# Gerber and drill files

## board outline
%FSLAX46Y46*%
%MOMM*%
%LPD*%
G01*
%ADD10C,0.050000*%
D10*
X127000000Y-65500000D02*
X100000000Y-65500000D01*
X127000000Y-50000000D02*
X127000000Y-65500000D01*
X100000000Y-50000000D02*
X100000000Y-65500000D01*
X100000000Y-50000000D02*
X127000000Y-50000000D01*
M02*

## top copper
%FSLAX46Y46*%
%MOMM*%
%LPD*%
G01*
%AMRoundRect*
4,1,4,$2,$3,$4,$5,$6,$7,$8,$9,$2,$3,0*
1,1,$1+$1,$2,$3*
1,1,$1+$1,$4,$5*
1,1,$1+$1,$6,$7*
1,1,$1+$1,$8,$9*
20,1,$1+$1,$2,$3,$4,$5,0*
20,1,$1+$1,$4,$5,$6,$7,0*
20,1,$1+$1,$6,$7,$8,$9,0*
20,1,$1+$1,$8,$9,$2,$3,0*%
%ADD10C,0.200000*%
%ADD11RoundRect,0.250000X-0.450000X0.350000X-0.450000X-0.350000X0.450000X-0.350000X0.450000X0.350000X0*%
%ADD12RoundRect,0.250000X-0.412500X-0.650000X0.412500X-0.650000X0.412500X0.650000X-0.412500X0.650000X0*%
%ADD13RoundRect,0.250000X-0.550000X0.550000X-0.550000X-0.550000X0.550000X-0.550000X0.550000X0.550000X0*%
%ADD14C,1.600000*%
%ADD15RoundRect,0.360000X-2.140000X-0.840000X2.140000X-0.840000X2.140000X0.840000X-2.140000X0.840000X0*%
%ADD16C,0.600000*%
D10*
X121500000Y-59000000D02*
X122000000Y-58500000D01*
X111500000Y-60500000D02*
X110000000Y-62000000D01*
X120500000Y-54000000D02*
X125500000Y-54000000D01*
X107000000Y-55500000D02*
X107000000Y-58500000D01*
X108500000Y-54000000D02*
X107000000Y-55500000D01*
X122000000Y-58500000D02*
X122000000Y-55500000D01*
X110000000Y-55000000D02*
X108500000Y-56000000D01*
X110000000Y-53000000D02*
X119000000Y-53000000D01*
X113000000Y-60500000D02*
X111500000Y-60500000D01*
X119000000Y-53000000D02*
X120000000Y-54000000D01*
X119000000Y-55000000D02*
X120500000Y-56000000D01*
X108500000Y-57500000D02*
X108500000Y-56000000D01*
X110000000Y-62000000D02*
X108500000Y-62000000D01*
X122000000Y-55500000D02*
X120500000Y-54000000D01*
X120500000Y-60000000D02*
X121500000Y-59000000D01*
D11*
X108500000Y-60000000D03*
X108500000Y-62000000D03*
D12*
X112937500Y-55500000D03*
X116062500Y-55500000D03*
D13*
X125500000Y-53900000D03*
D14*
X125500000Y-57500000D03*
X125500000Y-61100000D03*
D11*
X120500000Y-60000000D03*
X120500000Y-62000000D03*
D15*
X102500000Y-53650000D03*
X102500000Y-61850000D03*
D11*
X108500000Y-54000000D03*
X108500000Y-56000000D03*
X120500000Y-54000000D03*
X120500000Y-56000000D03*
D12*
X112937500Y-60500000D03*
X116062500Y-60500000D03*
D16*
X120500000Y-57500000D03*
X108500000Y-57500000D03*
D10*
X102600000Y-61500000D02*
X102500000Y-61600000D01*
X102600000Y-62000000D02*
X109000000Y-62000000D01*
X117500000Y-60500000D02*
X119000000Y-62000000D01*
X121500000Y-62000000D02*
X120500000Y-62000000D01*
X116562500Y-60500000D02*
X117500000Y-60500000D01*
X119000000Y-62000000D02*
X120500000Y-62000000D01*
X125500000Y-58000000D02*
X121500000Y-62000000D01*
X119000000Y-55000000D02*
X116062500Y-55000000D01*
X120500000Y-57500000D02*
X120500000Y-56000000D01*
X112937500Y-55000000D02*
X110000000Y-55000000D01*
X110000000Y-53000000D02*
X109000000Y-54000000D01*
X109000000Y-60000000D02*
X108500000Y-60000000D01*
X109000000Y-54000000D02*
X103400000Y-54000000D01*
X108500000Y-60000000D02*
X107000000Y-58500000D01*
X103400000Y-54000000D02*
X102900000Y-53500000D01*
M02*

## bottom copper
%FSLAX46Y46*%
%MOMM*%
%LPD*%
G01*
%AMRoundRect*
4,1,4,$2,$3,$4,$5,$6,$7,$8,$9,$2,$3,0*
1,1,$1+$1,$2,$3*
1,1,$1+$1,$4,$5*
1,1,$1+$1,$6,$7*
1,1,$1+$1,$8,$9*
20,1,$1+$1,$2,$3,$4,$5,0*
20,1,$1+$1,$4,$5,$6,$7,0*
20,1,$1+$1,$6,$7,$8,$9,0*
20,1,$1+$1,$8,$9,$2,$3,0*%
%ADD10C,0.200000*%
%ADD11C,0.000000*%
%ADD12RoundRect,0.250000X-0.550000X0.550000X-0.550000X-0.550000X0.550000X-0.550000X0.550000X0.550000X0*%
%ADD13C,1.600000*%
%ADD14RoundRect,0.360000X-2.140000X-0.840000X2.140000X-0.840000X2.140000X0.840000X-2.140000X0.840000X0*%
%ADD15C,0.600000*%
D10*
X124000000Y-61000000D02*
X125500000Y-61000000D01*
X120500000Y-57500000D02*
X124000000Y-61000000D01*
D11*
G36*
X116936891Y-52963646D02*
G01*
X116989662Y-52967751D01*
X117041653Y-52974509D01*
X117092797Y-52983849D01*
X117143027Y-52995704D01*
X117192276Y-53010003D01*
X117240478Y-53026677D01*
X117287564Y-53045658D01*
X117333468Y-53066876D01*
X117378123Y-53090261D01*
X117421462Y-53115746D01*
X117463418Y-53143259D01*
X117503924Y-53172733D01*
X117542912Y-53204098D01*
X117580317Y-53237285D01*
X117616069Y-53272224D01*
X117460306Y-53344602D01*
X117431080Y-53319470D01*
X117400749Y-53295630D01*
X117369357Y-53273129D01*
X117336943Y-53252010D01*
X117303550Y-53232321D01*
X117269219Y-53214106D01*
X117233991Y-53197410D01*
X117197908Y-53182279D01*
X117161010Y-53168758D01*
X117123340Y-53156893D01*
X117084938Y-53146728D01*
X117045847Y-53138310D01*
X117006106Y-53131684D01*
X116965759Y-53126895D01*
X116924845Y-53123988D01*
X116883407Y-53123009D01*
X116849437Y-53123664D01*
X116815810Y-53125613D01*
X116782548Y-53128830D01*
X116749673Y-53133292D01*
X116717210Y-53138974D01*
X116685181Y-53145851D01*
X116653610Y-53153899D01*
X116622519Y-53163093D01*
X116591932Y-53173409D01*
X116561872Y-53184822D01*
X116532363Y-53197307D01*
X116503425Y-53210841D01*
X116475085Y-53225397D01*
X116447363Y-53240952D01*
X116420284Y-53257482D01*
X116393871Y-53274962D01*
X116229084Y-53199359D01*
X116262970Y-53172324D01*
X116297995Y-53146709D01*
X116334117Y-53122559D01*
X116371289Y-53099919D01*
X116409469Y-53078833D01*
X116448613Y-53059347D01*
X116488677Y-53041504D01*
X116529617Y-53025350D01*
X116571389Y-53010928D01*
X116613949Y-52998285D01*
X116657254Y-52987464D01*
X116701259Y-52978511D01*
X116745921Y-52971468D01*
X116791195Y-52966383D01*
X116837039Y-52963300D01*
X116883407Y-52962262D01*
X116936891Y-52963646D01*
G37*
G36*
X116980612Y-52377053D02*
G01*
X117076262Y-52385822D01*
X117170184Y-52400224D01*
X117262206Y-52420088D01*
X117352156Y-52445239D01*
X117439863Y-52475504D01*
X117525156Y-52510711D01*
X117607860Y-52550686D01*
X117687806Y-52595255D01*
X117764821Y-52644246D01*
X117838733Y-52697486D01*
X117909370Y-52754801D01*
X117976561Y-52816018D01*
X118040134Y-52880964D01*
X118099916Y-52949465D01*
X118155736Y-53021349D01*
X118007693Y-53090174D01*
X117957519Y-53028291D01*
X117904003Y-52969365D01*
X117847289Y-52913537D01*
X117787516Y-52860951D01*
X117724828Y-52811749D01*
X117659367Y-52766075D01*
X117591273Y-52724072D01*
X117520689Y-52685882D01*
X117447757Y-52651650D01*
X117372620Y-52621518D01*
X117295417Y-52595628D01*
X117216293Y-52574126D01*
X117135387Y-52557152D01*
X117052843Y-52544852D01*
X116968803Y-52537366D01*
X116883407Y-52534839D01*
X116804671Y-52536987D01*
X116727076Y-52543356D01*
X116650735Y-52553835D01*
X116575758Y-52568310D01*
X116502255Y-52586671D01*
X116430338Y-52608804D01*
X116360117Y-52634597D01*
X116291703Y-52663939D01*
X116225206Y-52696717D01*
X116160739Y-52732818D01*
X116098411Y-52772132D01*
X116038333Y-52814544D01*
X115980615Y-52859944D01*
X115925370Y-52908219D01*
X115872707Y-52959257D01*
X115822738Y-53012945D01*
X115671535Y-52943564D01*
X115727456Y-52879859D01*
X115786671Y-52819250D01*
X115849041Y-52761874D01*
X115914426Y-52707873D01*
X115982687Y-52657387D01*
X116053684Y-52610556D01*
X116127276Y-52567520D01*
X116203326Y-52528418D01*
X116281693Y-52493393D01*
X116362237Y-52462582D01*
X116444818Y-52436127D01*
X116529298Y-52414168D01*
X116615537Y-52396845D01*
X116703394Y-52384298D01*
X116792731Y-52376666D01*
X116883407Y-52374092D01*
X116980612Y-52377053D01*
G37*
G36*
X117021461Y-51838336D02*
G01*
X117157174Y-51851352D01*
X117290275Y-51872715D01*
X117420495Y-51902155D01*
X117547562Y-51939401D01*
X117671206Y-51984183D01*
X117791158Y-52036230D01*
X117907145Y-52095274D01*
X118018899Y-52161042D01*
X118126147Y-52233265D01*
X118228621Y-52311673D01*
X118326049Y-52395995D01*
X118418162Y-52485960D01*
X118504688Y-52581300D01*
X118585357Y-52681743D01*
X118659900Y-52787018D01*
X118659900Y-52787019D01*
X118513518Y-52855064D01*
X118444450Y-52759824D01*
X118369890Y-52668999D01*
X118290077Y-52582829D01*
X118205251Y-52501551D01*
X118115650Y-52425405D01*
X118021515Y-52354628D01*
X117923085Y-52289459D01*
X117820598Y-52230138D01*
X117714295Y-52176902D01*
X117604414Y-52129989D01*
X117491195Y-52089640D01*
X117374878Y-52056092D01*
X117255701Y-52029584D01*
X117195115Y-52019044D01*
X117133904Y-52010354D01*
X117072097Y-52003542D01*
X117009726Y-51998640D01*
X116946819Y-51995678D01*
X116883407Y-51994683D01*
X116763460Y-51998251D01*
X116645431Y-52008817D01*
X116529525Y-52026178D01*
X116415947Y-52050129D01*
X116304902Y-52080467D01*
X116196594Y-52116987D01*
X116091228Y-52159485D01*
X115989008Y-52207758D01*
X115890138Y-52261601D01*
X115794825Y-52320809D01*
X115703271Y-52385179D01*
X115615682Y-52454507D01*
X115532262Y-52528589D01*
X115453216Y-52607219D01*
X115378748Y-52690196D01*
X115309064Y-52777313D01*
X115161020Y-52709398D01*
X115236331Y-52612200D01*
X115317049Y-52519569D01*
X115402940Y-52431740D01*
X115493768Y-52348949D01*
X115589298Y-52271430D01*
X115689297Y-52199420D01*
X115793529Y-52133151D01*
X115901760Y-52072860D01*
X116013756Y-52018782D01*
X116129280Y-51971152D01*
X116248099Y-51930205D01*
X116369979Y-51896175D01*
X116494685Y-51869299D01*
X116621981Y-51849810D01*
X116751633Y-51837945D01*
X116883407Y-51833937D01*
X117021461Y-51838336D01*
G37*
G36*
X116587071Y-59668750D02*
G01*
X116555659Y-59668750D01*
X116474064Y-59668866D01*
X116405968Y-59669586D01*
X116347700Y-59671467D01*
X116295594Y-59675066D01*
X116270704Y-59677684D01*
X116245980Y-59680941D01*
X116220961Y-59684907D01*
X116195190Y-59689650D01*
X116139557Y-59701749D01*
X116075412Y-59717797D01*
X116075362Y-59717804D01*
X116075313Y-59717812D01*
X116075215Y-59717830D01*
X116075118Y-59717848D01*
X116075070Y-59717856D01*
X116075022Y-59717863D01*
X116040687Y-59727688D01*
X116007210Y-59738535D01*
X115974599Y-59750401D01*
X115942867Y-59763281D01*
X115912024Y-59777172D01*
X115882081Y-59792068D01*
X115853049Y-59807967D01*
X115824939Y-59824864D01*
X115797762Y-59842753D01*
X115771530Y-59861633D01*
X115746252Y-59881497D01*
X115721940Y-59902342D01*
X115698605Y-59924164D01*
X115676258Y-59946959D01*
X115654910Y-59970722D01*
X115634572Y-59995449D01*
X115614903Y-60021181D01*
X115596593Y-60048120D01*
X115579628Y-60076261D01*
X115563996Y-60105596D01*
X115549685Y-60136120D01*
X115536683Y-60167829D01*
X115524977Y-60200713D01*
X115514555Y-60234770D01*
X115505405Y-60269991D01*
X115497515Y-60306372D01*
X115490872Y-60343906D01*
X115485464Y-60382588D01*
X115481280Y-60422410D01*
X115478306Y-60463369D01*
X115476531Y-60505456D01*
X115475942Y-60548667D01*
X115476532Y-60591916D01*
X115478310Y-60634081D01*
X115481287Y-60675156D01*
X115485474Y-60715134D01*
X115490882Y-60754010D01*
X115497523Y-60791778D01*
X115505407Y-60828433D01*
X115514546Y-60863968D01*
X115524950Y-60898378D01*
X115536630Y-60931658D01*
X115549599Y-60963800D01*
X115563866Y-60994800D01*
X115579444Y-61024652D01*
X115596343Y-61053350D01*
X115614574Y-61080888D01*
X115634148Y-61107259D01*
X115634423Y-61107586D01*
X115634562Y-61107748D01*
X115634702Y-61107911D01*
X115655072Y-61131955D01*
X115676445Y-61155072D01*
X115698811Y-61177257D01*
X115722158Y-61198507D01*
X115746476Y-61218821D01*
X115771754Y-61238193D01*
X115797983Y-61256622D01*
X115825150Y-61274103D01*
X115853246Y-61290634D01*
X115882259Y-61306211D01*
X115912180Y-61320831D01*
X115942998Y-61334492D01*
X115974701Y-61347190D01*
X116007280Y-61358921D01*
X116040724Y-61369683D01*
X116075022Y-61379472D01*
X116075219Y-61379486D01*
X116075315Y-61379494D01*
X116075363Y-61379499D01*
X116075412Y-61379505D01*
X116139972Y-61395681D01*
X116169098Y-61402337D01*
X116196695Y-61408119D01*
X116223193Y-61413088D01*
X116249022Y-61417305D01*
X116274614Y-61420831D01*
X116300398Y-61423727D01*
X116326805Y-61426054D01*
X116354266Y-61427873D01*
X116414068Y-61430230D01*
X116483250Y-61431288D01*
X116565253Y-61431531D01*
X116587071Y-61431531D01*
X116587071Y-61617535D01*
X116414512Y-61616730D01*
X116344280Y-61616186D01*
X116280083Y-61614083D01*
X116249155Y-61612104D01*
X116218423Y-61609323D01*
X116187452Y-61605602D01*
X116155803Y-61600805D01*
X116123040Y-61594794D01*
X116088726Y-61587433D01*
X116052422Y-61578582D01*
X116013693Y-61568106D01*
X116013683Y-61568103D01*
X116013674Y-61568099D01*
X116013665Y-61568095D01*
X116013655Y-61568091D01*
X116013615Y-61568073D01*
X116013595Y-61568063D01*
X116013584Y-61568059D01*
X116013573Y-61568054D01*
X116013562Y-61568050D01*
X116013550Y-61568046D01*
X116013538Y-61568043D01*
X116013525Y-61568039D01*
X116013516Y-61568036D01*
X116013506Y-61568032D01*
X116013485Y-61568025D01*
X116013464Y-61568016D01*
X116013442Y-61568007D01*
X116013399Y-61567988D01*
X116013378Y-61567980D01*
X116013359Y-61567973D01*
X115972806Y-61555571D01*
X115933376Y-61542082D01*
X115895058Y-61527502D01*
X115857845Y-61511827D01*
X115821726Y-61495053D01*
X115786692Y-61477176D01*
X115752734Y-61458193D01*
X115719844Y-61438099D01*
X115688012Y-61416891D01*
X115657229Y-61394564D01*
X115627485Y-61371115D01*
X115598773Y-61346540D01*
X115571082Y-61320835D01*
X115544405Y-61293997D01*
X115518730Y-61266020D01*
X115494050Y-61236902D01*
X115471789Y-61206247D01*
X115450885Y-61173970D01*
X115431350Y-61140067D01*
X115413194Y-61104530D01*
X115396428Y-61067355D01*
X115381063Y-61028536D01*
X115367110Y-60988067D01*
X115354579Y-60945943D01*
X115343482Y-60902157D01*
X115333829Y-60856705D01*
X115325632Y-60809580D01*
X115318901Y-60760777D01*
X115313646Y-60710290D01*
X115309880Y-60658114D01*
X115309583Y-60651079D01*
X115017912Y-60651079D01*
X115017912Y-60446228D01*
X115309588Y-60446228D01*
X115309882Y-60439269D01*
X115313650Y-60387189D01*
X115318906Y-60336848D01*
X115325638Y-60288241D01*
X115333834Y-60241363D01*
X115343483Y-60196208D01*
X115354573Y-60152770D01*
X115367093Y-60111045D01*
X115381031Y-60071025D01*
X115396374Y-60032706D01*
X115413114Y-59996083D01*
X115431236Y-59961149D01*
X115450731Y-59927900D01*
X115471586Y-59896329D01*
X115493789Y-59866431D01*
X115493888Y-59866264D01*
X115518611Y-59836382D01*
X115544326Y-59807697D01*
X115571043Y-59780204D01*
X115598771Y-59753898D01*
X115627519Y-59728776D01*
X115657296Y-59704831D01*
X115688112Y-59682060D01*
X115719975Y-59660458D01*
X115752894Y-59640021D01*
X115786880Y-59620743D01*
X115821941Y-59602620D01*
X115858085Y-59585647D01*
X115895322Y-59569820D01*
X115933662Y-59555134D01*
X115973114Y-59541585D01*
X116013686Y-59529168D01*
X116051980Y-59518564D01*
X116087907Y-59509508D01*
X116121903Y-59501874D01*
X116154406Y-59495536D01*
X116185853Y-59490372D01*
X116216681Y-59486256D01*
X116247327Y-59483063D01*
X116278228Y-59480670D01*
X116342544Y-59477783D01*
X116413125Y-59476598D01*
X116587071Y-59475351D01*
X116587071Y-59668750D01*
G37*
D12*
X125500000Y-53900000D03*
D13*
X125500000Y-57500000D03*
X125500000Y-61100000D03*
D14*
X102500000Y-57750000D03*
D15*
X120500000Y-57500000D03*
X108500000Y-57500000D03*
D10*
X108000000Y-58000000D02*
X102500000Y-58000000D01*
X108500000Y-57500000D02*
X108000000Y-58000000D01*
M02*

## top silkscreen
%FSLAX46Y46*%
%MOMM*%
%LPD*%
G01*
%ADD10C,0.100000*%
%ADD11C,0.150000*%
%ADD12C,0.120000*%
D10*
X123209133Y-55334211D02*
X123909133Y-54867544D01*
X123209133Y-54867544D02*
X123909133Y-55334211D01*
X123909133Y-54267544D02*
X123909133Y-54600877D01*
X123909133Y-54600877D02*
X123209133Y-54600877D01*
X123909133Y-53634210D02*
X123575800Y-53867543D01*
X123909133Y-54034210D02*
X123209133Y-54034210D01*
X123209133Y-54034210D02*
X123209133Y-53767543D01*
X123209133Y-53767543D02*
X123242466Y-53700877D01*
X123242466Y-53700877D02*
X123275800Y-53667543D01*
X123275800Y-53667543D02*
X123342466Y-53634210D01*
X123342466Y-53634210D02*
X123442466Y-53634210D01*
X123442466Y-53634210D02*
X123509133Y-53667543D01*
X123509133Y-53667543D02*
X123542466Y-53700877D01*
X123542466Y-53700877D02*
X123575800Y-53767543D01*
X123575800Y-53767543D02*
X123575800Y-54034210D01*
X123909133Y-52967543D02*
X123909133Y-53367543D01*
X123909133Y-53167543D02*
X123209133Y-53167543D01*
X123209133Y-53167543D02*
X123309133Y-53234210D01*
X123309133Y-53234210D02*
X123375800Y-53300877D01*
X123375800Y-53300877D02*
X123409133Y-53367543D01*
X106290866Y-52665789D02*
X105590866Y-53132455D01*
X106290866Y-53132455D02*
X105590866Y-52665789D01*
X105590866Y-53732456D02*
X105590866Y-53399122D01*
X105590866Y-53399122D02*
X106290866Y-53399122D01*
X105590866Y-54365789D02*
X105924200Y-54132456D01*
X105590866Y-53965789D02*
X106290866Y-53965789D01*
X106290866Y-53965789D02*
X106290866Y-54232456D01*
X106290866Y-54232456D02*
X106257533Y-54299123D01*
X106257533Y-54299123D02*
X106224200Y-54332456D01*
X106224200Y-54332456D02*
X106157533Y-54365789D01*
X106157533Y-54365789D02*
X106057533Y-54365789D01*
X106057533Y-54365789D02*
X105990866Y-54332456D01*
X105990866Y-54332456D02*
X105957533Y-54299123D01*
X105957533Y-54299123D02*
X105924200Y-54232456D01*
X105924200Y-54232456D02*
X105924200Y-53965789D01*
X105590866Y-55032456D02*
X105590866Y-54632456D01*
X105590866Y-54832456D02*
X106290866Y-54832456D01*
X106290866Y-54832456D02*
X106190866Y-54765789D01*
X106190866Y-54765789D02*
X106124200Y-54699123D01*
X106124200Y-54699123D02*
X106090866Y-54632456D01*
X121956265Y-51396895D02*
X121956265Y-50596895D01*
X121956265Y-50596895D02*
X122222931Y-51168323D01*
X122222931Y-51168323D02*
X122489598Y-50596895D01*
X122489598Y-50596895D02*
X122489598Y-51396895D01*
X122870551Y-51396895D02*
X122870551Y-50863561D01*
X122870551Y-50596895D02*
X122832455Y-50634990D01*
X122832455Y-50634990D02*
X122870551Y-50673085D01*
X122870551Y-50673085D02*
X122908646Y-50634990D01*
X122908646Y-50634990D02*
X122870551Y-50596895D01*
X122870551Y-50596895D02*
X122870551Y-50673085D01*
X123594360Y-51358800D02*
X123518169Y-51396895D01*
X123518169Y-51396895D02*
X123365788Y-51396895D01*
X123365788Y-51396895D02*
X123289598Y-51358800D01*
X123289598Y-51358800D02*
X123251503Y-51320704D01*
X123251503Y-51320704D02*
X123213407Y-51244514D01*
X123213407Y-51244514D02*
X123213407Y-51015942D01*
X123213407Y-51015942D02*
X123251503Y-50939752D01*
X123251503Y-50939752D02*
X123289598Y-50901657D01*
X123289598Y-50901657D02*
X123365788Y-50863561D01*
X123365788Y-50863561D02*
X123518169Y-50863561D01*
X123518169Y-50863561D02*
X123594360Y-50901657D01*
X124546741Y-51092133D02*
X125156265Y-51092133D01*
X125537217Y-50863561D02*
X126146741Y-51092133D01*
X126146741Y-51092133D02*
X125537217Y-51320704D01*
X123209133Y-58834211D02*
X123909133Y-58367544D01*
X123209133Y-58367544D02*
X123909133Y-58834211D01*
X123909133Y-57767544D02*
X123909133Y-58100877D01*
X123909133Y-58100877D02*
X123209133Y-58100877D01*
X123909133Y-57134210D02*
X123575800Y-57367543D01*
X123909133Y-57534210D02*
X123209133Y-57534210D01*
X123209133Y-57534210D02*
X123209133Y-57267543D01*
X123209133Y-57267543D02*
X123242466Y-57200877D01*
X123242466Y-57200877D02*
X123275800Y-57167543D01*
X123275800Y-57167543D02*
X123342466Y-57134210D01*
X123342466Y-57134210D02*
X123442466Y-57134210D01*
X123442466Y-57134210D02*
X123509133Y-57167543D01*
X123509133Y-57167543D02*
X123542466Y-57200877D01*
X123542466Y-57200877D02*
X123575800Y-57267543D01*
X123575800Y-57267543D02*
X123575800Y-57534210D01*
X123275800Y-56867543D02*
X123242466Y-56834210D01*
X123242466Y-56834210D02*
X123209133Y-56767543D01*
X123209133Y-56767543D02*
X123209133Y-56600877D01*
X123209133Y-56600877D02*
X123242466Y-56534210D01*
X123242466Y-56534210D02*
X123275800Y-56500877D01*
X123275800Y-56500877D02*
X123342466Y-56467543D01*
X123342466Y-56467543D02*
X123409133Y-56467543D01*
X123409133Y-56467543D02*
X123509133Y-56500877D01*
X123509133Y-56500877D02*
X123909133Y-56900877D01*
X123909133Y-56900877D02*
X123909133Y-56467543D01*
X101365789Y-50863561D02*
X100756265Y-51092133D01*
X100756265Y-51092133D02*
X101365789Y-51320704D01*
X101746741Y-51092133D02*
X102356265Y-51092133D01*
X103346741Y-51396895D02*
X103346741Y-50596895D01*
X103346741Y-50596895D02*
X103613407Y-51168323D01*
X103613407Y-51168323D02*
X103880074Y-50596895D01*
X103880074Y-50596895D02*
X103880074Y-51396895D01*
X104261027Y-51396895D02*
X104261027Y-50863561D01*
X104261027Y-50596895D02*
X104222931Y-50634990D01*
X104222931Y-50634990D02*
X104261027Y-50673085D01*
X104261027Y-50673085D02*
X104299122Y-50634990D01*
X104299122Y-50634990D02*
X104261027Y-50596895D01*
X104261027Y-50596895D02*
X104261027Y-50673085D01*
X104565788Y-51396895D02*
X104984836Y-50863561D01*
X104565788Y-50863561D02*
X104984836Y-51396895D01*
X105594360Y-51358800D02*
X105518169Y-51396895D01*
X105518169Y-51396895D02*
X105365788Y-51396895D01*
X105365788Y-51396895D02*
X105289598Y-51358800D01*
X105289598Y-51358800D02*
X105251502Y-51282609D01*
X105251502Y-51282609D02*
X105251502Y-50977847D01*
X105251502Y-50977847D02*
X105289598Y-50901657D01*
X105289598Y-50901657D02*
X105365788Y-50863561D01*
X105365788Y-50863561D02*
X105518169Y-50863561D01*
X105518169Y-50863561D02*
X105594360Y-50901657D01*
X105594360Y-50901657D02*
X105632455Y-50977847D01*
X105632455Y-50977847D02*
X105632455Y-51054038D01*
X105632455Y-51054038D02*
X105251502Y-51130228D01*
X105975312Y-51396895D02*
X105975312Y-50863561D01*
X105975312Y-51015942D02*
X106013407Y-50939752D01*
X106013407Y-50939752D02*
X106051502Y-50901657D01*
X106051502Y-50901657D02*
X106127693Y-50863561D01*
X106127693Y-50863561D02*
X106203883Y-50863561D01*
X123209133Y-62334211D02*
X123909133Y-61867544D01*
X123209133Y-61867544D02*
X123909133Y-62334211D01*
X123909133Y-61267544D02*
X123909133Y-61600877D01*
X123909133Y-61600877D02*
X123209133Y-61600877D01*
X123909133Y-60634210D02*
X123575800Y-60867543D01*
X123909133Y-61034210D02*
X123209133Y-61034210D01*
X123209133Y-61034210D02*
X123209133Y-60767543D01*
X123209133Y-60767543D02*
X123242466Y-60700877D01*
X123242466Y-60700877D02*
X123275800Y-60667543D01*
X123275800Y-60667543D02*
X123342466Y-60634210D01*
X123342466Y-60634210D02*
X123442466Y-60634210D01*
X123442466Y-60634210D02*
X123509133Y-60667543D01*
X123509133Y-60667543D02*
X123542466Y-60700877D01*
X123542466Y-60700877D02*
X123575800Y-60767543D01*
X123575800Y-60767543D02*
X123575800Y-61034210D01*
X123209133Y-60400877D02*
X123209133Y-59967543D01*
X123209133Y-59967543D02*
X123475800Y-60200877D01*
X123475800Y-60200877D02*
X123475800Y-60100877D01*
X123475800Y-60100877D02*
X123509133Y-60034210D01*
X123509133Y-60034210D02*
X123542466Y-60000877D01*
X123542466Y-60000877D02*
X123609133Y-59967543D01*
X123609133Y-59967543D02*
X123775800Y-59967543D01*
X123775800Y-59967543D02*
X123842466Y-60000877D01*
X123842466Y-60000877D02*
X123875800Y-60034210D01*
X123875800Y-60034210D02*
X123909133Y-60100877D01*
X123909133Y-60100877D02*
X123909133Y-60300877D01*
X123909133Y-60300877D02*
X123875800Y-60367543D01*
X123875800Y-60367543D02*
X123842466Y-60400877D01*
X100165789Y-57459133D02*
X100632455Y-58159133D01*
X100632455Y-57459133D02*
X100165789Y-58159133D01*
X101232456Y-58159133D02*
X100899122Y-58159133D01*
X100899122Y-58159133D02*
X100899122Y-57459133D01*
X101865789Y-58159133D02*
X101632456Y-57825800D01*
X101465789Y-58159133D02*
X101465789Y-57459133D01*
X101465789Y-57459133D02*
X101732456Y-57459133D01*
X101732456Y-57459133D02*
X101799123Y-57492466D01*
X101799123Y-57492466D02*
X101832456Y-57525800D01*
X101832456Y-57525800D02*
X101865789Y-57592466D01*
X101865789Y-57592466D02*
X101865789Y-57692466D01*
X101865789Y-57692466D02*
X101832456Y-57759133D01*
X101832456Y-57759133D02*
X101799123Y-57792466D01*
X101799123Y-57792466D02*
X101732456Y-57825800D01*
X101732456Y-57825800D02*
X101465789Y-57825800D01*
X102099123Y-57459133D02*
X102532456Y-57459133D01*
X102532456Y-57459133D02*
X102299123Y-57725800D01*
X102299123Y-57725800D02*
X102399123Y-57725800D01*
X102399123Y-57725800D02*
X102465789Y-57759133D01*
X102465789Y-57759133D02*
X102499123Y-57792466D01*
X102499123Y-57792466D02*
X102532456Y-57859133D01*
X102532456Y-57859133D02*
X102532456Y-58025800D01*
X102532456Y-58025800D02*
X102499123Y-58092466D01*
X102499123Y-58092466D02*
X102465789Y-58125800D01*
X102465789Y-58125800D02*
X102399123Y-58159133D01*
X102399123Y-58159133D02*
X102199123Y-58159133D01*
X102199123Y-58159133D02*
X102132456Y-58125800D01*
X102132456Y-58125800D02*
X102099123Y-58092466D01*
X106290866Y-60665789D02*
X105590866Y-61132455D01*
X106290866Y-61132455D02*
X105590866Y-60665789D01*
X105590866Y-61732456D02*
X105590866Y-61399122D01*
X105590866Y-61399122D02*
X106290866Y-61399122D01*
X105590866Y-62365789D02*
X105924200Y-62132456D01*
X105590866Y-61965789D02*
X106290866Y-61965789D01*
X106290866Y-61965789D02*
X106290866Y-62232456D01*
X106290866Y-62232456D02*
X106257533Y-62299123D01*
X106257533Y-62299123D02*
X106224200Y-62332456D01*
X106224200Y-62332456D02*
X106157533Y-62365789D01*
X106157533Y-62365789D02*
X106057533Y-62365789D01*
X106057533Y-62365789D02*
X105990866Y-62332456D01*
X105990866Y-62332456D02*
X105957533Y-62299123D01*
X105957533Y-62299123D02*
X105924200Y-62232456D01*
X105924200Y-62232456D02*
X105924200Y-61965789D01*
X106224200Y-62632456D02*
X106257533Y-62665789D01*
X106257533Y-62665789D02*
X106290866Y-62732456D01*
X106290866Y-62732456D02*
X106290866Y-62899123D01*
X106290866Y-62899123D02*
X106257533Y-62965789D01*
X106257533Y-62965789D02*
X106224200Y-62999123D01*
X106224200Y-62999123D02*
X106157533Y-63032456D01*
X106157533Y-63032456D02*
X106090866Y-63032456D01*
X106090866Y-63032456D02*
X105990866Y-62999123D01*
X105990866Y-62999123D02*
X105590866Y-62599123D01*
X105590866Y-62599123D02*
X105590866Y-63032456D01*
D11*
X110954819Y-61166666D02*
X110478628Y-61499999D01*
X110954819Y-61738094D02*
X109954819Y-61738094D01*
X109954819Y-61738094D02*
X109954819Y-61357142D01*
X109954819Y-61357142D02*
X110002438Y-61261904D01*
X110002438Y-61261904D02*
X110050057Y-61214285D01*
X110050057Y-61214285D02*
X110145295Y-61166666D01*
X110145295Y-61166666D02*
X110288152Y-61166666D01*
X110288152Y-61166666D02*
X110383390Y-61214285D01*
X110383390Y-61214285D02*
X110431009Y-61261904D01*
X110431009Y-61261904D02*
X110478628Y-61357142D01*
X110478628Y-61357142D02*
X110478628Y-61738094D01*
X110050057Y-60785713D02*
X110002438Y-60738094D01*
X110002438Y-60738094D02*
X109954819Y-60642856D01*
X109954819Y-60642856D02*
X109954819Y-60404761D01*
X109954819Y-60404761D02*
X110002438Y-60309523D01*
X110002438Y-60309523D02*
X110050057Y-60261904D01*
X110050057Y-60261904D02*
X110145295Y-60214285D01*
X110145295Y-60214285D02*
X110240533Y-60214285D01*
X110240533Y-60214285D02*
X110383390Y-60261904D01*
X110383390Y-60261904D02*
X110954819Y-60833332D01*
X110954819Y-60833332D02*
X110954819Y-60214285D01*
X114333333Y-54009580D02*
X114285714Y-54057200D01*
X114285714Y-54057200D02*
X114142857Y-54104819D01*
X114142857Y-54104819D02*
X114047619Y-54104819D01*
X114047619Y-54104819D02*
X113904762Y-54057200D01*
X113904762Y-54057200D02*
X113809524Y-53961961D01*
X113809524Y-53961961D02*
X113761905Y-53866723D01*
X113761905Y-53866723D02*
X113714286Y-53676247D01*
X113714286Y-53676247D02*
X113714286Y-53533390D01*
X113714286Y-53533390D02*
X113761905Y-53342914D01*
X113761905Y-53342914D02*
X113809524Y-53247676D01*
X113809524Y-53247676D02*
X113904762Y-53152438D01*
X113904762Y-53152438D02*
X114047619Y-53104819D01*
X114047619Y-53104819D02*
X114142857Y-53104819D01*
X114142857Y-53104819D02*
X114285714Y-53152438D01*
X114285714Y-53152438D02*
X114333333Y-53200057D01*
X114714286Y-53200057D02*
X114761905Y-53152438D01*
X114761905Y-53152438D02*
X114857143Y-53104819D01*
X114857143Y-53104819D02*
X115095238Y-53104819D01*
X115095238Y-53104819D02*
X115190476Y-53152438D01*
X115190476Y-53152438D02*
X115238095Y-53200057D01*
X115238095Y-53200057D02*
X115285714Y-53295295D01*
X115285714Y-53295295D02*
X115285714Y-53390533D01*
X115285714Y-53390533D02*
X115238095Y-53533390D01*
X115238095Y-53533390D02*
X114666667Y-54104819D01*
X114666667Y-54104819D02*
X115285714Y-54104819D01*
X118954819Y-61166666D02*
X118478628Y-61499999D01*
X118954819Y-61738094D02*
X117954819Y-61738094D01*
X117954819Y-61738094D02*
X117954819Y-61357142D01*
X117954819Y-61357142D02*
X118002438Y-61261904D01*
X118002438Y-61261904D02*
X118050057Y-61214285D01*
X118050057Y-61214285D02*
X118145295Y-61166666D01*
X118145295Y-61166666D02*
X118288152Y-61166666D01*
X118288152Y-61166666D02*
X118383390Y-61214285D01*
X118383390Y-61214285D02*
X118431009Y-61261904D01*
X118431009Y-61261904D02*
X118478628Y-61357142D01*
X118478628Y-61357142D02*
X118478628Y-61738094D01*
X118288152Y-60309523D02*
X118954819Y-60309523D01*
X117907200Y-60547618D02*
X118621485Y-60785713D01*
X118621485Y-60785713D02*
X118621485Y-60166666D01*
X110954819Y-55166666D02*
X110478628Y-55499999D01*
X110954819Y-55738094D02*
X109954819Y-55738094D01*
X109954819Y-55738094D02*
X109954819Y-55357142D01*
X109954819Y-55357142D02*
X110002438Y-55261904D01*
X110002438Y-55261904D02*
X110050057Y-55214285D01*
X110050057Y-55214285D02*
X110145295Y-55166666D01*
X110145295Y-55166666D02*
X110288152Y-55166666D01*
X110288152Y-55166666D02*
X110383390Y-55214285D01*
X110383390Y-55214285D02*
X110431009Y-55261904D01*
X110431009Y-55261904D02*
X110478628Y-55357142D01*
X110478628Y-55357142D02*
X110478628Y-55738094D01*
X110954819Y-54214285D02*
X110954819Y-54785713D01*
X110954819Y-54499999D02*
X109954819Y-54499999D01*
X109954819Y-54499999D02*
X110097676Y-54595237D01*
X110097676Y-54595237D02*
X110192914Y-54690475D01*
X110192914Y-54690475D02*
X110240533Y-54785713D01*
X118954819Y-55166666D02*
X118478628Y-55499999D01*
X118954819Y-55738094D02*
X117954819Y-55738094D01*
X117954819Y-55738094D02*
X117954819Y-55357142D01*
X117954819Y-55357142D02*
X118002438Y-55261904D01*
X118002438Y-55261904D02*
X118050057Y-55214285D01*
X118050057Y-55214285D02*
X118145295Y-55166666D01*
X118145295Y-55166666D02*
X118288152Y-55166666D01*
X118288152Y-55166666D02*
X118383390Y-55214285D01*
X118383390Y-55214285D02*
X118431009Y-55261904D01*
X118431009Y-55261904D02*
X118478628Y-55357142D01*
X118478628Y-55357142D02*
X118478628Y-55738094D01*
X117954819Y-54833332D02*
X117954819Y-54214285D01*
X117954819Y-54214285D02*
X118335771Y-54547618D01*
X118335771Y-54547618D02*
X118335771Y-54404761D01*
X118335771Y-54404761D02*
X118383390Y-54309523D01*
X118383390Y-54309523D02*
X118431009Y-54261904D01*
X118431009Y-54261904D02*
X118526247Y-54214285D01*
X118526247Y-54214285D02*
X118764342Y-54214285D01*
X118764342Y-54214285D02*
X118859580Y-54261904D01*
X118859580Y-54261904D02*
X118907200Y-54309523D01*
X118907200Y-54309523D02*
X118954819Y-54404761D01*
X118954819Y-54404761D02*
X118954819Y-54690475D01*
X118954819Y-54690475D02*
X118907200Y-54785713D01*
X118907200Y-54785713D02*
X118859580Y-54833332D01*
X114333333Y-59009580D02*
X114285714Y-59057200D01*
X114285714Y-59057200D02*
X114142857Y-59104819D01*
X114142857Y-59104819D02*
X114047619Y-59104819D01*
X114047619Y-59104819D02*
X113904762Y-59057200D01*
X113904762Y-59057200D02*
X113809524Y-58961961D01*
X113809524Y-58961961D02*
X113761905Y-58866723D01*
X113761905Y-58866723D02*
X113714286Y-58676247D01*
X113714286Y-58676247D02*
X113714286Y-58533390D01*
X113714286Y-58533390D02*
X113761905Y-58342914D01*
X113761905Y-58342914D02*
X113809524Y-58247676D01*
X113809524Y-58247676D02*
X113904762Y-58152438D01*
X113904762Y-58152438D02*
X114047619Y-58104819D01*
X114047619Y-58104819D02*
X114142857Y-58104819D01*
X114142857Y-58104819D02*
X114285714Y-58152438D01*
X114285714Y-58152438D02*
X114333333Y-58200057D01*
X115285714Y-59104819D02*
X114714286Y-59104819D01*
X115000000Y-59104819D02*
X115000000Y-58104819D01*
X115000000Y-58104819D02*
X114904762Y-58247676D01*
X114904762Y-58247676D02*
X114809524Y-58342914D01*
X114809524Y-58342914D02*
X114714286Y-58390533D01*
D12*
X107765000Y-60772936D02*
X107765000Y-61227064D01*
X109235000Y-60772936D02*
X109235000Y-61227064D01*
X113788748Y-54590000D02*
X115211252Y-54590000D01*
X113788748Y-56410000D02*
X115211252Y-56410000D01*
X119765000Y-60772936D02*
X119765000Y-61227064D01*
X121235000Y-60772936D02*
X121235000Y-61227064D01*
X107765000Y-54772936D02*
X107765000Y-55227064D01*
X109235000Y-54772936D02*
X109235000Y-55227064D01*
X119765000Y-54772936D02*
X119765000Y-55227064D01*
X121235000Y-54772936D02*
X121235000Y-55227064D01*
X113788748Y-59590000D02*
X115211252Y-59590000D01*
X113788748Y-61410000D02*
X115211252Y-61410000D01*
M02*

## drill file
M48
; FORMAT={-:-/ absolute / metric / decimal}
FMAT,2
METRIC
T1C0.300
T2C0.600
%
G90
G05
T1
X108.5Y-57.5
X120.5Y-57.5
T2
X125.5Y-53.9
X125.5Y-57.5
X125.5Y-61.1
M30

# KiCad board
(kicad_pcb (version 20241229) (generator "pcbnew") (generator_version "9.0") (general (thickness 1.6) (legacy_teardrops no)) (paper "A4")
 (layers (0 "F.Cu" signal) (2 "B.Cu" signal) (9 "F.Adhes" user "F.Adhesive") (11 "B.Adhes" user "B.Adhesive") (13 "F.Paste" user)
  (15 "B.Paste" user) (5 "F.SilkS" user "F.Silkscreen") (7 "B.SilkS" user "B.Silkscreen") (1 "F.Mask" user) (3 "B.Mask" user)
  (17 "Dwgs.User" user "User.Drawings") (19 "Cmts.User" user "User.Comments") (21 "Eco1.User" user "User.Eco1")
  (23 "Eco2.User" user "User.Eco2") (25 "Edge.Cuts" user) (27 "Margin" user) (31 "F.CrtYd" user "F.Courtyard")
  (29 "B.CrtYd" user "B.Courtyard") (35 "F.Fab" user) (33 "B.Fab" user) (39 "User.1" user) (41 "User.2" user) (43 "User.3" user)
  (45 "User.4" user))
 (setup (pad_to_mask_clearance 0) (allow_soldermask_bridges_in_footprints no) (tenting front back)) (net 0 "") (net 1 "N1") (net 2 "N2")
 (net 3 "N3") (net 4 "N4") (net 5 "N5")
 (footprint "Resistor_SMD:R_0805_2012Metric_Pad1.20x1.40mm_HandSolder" (layer "F.Cu") (at 108.5 61 -90)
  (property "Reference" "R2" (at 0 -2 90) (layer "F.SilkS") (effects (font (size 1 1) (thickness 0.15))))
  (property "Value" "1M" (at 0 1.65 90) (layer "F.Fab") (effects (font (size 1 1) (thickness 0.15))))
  (fp_line (start -0.227064 0.735) (end 0.227064 0.735) (stroke (width 0.12) (type solid)) (layer "F.SilkS"))
  (fp_line (start -0.227064 -0.735) (end 0.227064 -0.735) (stroke (width 0.12) (type solid)) (layer "F.SilkS"))
  (pad "1" smd roundrect (at -1 0 270) (size 1.2 1.4) (layers "F.Cu" "F.Mask" "F.Paste") (roundrect_rratio 0.208333) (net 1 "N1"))
  (pad "2" smd roundrect (at 1 0 270) (size 1.2 1.4) (layers "F.Cu" "F.Mask" "F.Paste") (roundrect_rratio 0.208333) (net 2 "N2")))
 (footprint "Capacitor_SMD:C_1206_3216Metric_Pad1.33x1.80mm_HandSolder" (layer "F.Cu") (at 114.5 55.5)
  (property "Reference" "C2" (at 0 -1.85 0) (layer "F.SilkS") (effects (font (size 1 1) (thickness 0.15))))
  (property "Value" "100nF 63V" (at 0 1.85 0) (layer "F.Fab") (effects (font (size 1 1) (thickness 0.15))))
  (fp_line (start -0.711252 -0.91) (end 0.711252 -0.91) (stroke (width 0.12) (type solid)) (layer "F.SilkS"))
  (fp_line (start -0.711252 0.91) (end 0.711252 0.91) (stroke (width 0.12) (type solid)) (layer "F.SilkS"))
  (pad "1" smd roundrect (at -1.5625 0) (size 1.325 1.8) (layers "F.Cu" "F.Mask" "F.Paste") (roundrect_rratio 0.188679) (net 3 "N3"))
  (pad "2" smd roundrect (at 1.5625 0) (size 1.325 1.8) (layers "F.Cu" "F.Mask" "F.Paste") (roundrect_rratio 0.188679) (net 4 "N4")))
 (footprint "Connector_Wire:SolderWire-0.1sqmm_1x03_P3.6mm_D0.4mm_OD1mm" (layer "F.Cu") (at 125.5 53.9 -90)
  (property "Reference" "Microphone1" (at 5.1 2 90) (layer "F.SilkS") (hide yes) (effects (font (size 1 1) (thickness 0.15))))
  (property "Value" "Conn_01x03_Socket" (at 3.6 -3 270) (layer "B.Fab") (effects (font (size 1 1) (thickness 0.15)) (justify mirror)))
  (pad "1" thru_hole roundrect (at 0 0 270) (size 1.6 1.6) (drill 0.6) (layers "*.Cu" "*.Mask") (remove_unused_layers no)
   (roundrect_rratio 0.15625) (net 1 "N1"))
  (pad "2" thru_hole circle (at 3.6 0 270) (size 1.6 1.6) (drill 0.6) (layers "*.Cu" "*.Mask") (remove_unused_layers no) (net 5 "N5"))
  (pad "3" thru_hole circle (at 7.2 0 270) (size 1.6 1.6) (drill 0.6) (layers "*.Cu" "*.Mask") (remove_unused_layers no) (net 4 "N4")))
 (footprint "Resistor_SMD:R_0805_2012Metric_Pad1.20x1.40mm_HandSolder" (layer "F.Cu") (at 120.5 61 -90)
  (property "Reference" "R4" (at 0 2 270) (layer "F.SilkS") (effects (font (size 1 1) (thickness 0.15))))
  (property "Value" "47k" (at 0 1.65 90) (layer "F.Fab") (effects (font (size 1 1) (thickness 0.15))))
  (fp_line (start -0.227064 0.735) (end 0.227064 0.735) (stroke (width 0.12) (type solid)) (layer "F.SilkS"))
  (fp_line (start -0.227064 -0.735) (end 0.227064 -0.735) (stroke (width 0.12) (type solid)) (layer "F.SilkS"))
  (pad "1" smd roundrect (at -1 0 270) (size 1.2 1.4) (layers "F.Cu" "F.Mask" "F.Paste") (roundrect_rratio 0.208333) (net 1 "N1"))
  (pad "2" smd roundrect (at 1 0 270) (size 1.2 1.4) (layers "F.Cu" "F.Mask" "F.Paste") (roundrect_rratio 0.208333) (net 5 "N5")))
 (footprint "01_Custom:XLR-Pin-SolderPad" (layer "F.Cu") (at 102.5 57.75)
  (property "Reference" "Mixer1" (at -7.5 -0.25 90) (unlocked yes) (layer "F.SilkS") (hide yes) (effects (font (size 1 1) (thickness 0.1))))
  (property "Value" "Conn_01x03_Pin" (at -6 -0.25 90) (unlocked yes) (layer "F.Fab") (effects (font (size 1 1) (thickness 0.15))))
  (pad "1" smd roundrect (at 0 -4.1) (size 5 2.4) (layers "F.Cu" "F.Mask") (roundrect_rratio 0.15) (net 1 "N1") (solder_mask_margin 0.1))
  (pad "2" smd roundrect (at 0 4.1) (size 5 2.4) (layers "F.Cu" "F.Mask") (roundrect_rratio 0.15) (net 2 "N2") (solder_mask_margin 0.1))
  (pad "3" smd roundrect (at 0 0) (size 5 2.4) (layers "B.Cu" "B.Mask") (roundrect_rratio 0.15) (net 3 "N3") (solder_mask_margin 0.1)))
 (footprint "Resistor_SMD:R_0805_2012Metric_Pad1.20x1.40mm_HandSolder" (layer "F.Cu") (at 108.5 55 -90)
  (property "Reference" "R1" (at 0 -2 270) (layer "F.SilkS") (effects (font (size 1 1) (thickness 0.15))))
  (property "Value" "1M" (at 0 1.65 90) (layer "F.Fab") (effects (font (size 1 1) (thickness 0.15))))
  (fp_line (start -0.227064 0.735) (end 0.227064 0.735) (stroke (width 0.12) (type solid)) (layer "F.SilkS"))
  (fp_line (start -0.227064 -0.735) (end 0.227064 -0.735) (stroke (width 0.12) (type solid)) (layer "F.SilkS"))
  (pad "1" smd roundrect (at -1 0 270) (size 1.2 1.4) (layers "F.Cu" "F.Mask" "F.Paste") (roundrect_rratio 0.208333) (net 1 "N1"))
  (pad "2" smd roundrect (at 1 0 270) (size 1.2 1.4) (layers "F.Cu" "F.Mask" "F.Paste") (roundrect_rratio 0.208333) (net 3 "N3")))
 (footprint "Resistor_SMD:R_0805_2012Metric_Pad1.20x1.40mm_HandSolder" (layer "F.Cu") (at 120.5 55 -90)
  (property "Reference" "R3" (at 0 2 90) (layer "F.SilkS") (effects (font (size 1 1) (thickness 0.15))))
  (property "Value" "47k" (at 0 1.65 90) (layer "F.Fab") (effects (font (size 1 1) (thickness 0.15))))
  (fp_line (start -0.227064 0.735) (end 0.227064 0.735) (stroke (width 0.12) (type solid)) (layer "F.SilkS"))
  (fp_line (start -0.227064 -0.735) (end 0.227064 -0.735) (stroke (width 0.12) (type solid)) (layer "F.SilkS"))
  (pad "1" smd roundrect (at -1 0 270) (size 1.2 1.4) (layers "F.Cu" "F.Mask" "F.Paste") (roundrect_rratio 0.208333) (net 1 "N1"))
  (pad "2" smd roundrect (at 1 0 270) (size 1.2 1.4) (layers "F.Cu" "F.Mask" "F.Paste") (roundrect_rratio 0.208333) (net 4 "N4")))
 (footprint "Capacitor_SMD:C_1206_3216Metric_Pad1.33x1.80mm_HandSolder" (layer "F.Cu") (at 114.5 60.5)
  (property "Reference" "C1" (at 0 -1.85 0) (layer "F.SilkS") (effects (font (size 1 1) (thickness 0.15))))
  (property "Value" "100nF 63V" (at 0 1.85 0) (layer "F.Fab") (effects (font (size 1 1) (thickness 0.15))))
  (fp_line (start -0.711252 -0.91) (end 0.711252 -0.91) (stroke (width 0.12) (type solid)) (layer "F.SilkS"))
  (fp_line (start -0.711252 0.91) (end 0.711252 0.91) (stroke (width 0.12) (type solid)) (layer "F.SilkS"))
  (pad "1" smd roundrect (at -1.5625 0) (size 1.325 1.8) (layers "F.Cu" "F.Mask" "F.Paste") (roundrect_rratio 0.188679) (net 2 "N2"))
  (pad "2" smd roundrect (at 1.5625 0) (size 1.325 1.8) (layers "F.Cu" "F.Mask" "F.Paste") (roundrect_rratio 0.188679) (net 5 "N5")))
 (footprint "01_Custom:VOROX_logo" (layer "B.Cu") (at 115 66 90)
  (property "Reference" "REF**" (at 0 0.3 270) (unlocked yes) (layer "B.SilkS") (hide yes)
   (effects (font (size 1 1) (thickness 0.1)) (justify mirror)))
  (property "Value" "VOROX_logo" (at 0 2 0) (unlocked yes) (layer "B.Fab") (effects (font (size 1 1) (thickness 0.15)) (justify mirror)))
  (fp_poly
   (pts (xy 12.762715 2.580317) (xy 12.795902 2.542912) (xy 12.827267 2.503924) (xy 12.856741 2.463418) (xy 12.884254 2.421462)
    (xy 12.909739 2.378123) (xy 12.933124 2.333468) (xy 12.954342 2.287564) (xy 12.973323 2.240478) (xy 12.989997 2.192276)
    (xy 13.004296 2.143027) (xy 13.016151 2.092797) (xy 13.025491 2.041653) (xy 13.032249 1.989662) (xy 13.036354 1.936891)
    (xy 13.037738 1.883407) (xy 13.0367 1.837039) (xy 13.033617 1.791195) (xy 13.028532 1.745921) (xy 13.021489 1.701259)
    (xy 13.012536 1.657254) (xy 13.001715 1.613949) (xy 12.989072 1.571389) (xy 12.97465 1.529617) (xy 12.958496 1.488677)
    (xy 12.940653 1.448613) (xy 12.921167 1.409469) (xy 12.900081 1.371289) (xy 12.877441 1.334117) (xy 12.853291 1.297995)
    (xy 12.827676 1.26297) (xy 12.800641 1.229084) (xy 12.725038 1.393871) (xy 12.742518 1.420284) (xy 12.759048 1.447363)
    (xy 12.774603 1.475085) (xy 12.789159 1.503425) (xy 12.802693 1.532363) (xy 12.815178 1.561872) (xy 12.826591 1.591932)
    (xy 12.836907 1.622519) (xy 12.846101 1.65361) (xy 12.854149 1.685181) (xy 12.861026 1.71721) (xy 12.866708 1.749673)
    (xy 12.87117 1.782548) (xy 12.874387 1.81581) (xy 12.876336 1.849437) (xy 12.876991 1.883407) (xy 12.876012 1.924845)
    (xy 12.873105 1.965759) (xy 12.868316 2.006106) (xy 12.86169 2.045847) (xy 12.853272 2.084938) (xy 12.843107 2.12334)
    (xy 12.831242 2.16101) (xy 12.817721 2.197908) (xy 12.80259 2.233991) (xy 12.785894 2.269219) (xy 12.767679 2.30355)
    (xy 12.74799 2.336943) (xy 12.726871 2.369357) (xy 12.70437 2.400749) (xy 12.68053 2.43108) (xy 12.655398 2.460306)
    (xy 12.727776 2.616069))
   (stroke (width 0) (type solid)) (fill yes) (layer "B.Cu"))
  (fp_poly
   (pts (xy 13.050535 3.099916) (xy 13.119036 3.040134) (xy 13.183982 2.976561) (xy 13.245199 2.90937) (xy 13.302514 2.838733)
    (xy 13.355754 2.764821) (xy 13.404745 2.687806) (xy 13.449314 2.60786) (xy 13.489289 2.525156) (xy 13.524496 2.439863)
    (xy 13.554761 2.352156) (xy 13.579912 2.262206) (xy 13.599776 2.170184) (xy 13.614178 2.076262) (xy 13.622947 1.980612)
    (xy 13.625908 1.883407) (xy 13.623334 1.792731) (xy 13.615702 1.703394) (xy 13.603155 1.615537) (xy 13.585832 1.529298)
    (xy 13.563873 1.444818) (xy 13.537418 1.362237) (xy 13.506607 1.281693) (xy 13.471582 1.203326) (xy 13.43248 1.127276)
    (xy 13.389444 1.053684) (xy 13.342613 0.982687) (xy 13.292127 0.914426) (xy 13.238126 0.849041) (xy 13.18075 0.786671)
    (xy 13.120141 0.727456) (xy 13.056436 0.671535) (xy 12.987055 0.822738) (xy 13.040743 0.872707) (xy 13.091781 0.92537)
    (xy 13.140056 0.980615) (xy 13.185456 1.038333) (xy 13.227868 1.098411) (xy 13.267182 1.160739) (xy 13.303283 1.225206)
    (xy 13.336061 1.291703) (xy 13.365403 1.360117) (xy 13.391196 1.430338) (xy 13.413329 1.502255) (xy 13.43169 1.575758)
    (xy 13.446165 1.650735) (xy 13.456644 1.727076) (xy 13.463013 1.804671) (xy 13.465161 1.883407) (xy 13.462634 1.968803)
    (xy 13.455148 2.052843) (xy 13.442848 2.135387) (xy 13.425874 2.216293) (xy 13.404372 2.295417) (xy 13.378482 2.37262)
    (xy 13.34835 2.447757) (xy 13.314118 2.520689) (xy 13.275928 2.591273) (xy 13.233925 2.659367) (xy 13.188251 2.724828)
    (xy 13.139049 2.787516) (xy 13.086463 2.847289) (xy 13.030635 2.904003) (xy 12.971709 2.957519) (xy 12.909826 3.007693)
    (xy 12.978651 3.155736))
   (stroke (width 0) (type solid)) (fill yes) (layer "B.Cu"))
  (fp_poly
   (pts (xy 13.318257 3.585357) (xy 13.4187 3.504688) (xy 13.51404 3.418162) (xy 13.604005 3.326049) (xy 13.688327 3.228621)
    (xy 13.766735 3.126147) (xy 13.838958 3.018899) (xy 13.904726 2.907145) (xy 13.96377 2.791158) (xy 14.015817 2.671206)
    (xy 14.060599 2.547562) (xy 14.097845 2.420495) (xy 14.127285 2.290275) (xy 14.148648 2.157174) (xy 14.161664 2.021461)
    (xy 14.166063 1.883407) (xy 14.162055 1.751633) (xy 14.15019 1.621981) (xy 14.130701 1.494685) (xy 14.103825 1.369979)
    (xy 14.069795 1.248099) (xy 14.028848 1.12928) (xy 13.981218 1.013756) (xy 13.92714 0.90176) (xy 13.866849 0.793529)
    (xy 13.80058 0.689297) (xy 13.72857 0.589298) (xy 13.651051 0.493768) (xy 13.56826 0.40294) (xy 13.480431 0.317049)
    (xy 13.3878 0.236331) (xy 13.290602 0.16102) (xy 13.222687 0.309064) (xy 13.309804 0.378748) (xy 13.392781 0.453216)
    (xy 13.471411 0.532262) (xy 13.545493 0.615682) (xy 13.614821 0.703271) (xy 13.679191 0.794825) (xy 13.738399 0.890138)
    (xy 13.792242 0.989008) (xy 13.840515 1.091228) (xy 13.883013 1.196594) (xy 13.919533 1.304902) (xy 13.949871 1.415947)
    (xy 13.973822 1.529525) (xy 13.991183 1.645431) (xy 14.001749 1.76346) (xy 14.005317 1.883407) (xy 14.004322 1.946819)
    (xy 14.00136 2.009726) (xy 13.996458 2.072097) (xy 13.989646 2.133904) (xy 13.980956 2.195115) (xy 13.970416 2.255701)
    (xy 13.943908 2.374878) (xy 13.91036 2.491195) (xy 13.870011 2.604414) (xy 13.823098 2.714295) (xy 13.769862 2.820598)
    (xy 13.710541 2.923085) (xy 13.645372 3.021515) (xy 13.574595 3.11565) (xy 13.498449 3.205251) (xy 13.417171 3.290077)
    (xy 13.331001 3.36989) (xy 13.240176 3.44445) (xy 13.144936 3.513518) (xy 13.212981 3.6599) (xy 13.212982 3.6599))
   (stroke (width 0) (type solid)) (fill yes) (layer "B.Cu"))
  (fp_poly
   (pts (xy 4.568469 1.565253) (xy 4.568712 1.48325) (xy 4.56977 1.414068) (xy 4.572127 1.354266) (xy 4.573946 1.326805)
    (xy 4.576273 1.300398) (xy 4.579169 1.274614) (xy 4.582695 1.249022) (xy 4.586912 1.223193) (xy 4.591881 1.196695)
    (xy 4.597663 1.169098) (xy 4.604319 1.139972) (xy 4.620495 1.075412) (xy 4.620501 1.075363) (xy 4.620506 1.075315)
    (xy 4.620514 1.075219) (xy 4.620528 1.075022) (xy 4.630317 1.040724) (xy 4.641079 1.00728) (xy 4.65281 0.974701) (xy 4.665508 0.942998)
    (xy 4.679169 0.91218) (xy 4.693789 0.882259) (xy 4.709366 0.853246) (xy 4.725897 0.82515) (xy 4.743378 0.797983) (xy 4.761807 0.771754)
    (xy 4.781179 0.746476) (xy 4.801493 0.722158) (xy 4.822743 0.698811) (xy 4.844928 0.676445) (xy 4.868045 0.655072)
    (xy 4.892089 0.634702) (xy 4.892252 0.634562) (xy 4.892414 0.634423) (xy 4.892741 0.634148) (xy 4.919112 0.614574) (xy 4.94665 0.596343)
    (xy 4.975348 0.579444) (xy 5.0052 0.563866) (xy 5.0362 0.549599) (xy 5.068342 0.53663) (xy 5.101622 0.52495) (xy 5.136032 0.514546)
    (xy 5.171567 0.505407) (xy 5.208222 0.497523) (xy 5.24599 0.490882) (xy 5.284866 0.485474) (xy 5.324844 0.481287) (xy 5.365919 0.47831)
    (xy 5.408084 0.476532) (xy 5.451333 0.475942) (xy 5.494544 0.476531) (xy 5.536631 0.478306) (xy 5.57759 0.48128) (xy 5.617412 0.485464)
    (xy 5.656094 0.490872) (xy 5.693628 0.497515) (xy 5.730009 0.505405) (xy 5.76523 0.514555) (xy 5.799287 0.524977) (xy 5.832171 0.536683)
    (xy 5.86388 0.549685) (xy 5.894404 0.563996) (xy 5.923739 0.579628) (xy 5.95188 0.596593) (xy 5.978819 0.614903) (xy 6.004551 0.634572)
    (xy 6.029278 0.65491) (xy 6.053041 0.676258) (xy 6.075836 0.698605) (xy 6.097658 0.72194) (xy 6.118503 0.746252) (xy 6.138367 0.77153)
    (xy 6.157247 0.797762) (xy 6.175136 0.824939) (xy 6.192033 0.853049) (xy 6.207932 0.882081) (xy 6.222828 0.912024)
    (xy 6.236719 0.942867) (xy 6.249599 0.974599) (xy 6.261465 1.00721) (xy 6.272312 1.040687) (xy 6.282137 1.075022) (xy 6.282144 1.07507)
    (xy 6.282152 1.075118) (xy 6.28217 1.075215) (xy 6.282188 1.075313) (xy 6.282196 1.075362) (xy 6.282203 1.075412) (xy 6.298251 1.139557)
    (xy 6.31035 1.19519) (xy 6.315093 1.220961) (xy 6.319059 1.24598) (xy 6.322316 1.270704) (xy 6.324934 1.295594) (xy 6.328533 1.3477)
    (xy 6.330414 1.405968) (xy 6.331134 1.474064) (xy 6.33125 1.555659) (xy 6.33125 1.587071) (xy 6.524649 1.587071) (xy 6.523402 1.413125)
    (xy 6.522217 1.342544) (xy 6.51933 1.278228) (xy 6.516937 1.247327) (xy 6.513744 1.216681) (xy 6.509628 1.185853) (xy 6.504464 1.154406)
    (xy 6.498126 1.121903) (xy 6.490492 1.087907) (xy 6.481436 1.05198) (xy 6.470832 1.013686) (xy 6.458415 0.973114) (xy 6.444866 0.933662)
    (xy 6.43018 0.895322) (xy 6.414353 0.858085) (xy 6.39738 0.821941) (xy 6.379257 0.78688) (xy 6.359979 0.752894) (xy 6.339542 0.719975)
    (xy 6.31794 0.688112) (xy 6.295169 0.657296) (xy 6.271224 0.627519) (xy 6.246102 0.598771) (xy 6.219796 0.571043) (xy 6.192303 0.544326)
    (xy 6.163618 0.518611) (xy 6.133736 0.493888) (xy 6.133569 0.493789) (xy 6.103671 0.471586) (xy 6.0721 0.450731) (xy 6.038851 0.431236)
    (xy 6.003917 0.413114) (xy 5.967294 0.396374) (xy 5.928975 0.381031) (xy 5.888955 0.367093) (xy 5.84723 0.354573) (xy 5.803792 0.343483)
    (xy 5.758637 0.333834) (xy 5.711759 0.325638) (xy 5.663152 0.318906) (xy 5.612811 0.31365) (xy 5.560731 0.309882) (xy 5.553772 0.309588)
    (xy 5.553772 0.017912) (xy 5.348921 0.017912) (xy 5.348921 0.309583) (xy 5.341886 0.30988) (xy 5.28971 0.313646) (xy 5.239223 0.318901)
    (xy 5.19042 0.325632) (xy 5.143295 0.333829) (xy 5.097843 0.343482) (xy 5.054057 0.354579) (xy 5.011933 0.36711) (xy 4.971464 0.381063)
    (xy 4.932645 0.396428) (xy 4.89547 0.413194) (xy 4.859933 0.43135) (xy 4.82603 0.450885) (xy 4.793753 0.471789) (xy 4.763098 0.49405)
    (xy 4.73398 0.51873) (xy 4.706003 0.544405) (xy 4.679165 0.571082) (xy 4.65346 0.598773) (xy 4.628885 0.627485) (xy 4.605436 0.657229)
    (xy 4.583109 0.688012) (xy 4.561901 0.719844) (xy 4.541807 0.752734) (xy 4.522824 0.786692) (xy 4.504947 0.821726)
    (xy 4.488173 0.857845) (xy 4.472498 0.895058) (xy 4.457918 0.933376) (xy 4.444429 0.972806) (xy 4.432027 1.013359) (xy 4.43202 1.013378)
    (xy 4.432012 1.013399) (xy 4.431993 1.013442) (xy 4.431984 1.013464) (xy 4.431975 1.013485) (xy 4.431968 1.013506)
    (xy 4.431964 1.013516) (xy 4.431961 1.013525) (xy 4.431957 1.013538) (xy 4.431954 1.01355) (xy 4.43195 1.013562) (xy 4.431946 1.013573)
    (xy 4.431941 1.013584) (xy 4.431937 1.013595) (xy 4.431927 1.013615) (xy 4.431909 1.013655) (xy 4.431905 1.013665)
    (xy 4.431901 1.013674) (xy 4.431897 1.013683) (xy 4.431894 1.013693) (xy 4.421418 1.052422) (xy 4.412567 1.088726) (xy 4.405206 1.12304)
    (xy 4.399195 1.155803) (xy 4.394398 1.187452) (xy 4.390677 1.218423) (xy 4.387896 1.249155) (xy 4.385917 1.280083) (xy 4.383814 1.34428)
    (xy 4.38327 1.414512) (xy 4.382465 1.587071) (xy 4.568469 1.587071))
   (stroke (width 0) (type solid)) (fill yes) (layer "B.Cu")))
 (gr_line (start 121.5 59) (end 122 58.5) (stroke (width 0.2) (type default)) (layer "F.Cu") (net 1))
 (gr_line (start 111.5 60.5) (end 110 62) (stroke (width 0.2) (type default)) (layer "F.Cu") (net 2))
 (gr_line (start 120.5 54) (end 125.5 54) (stroke (width 0.2) (type default)) (layer "F.Cu") (net 1))
 (gr_line (start 107 55.5) (end 107 58.5) (stroke (width 0.2) (type default)) (layer "F.Cu") (net 1))
 (gr_line (start 108.5 54) (end 107 55.5) (stroke (width 0.2) (type default)) (layer "F.Cu") (net 1))
 (gr_line (start 122 58.5) (end 122 55.5) (stroke (width 0.2) (type default)) (layer "F.Cu") (net 1))
 (gr_line (start 110 55) (end 108.5 56) (stroke (width 0.2) (type default)) (layer "F.Cu") (net 3))
 (gr_line (start 110 53) (end 119 53) (stroke (width 0.2) (type default)) (layer "F.Cu") (net 1))
 (gr_line (start 113 60.5) (end 111.5 60.5) (stroke (width 0.2) (type default)) (layer "F.Cu") (net 2))
 (gr_line (start 119 53) (end 120 54) (stroke (width 0.2) (type default)) (layer "F.Cu") (net 1))
 (gr_line (start 119 55) (end 120.5 56) (stroke (width 0.2) (type default)) (layer "F.Cu") (net 4))
 (gr_line (start 108.5 57.5) (end 108.5 56) (stroke (width 0.2) (type default)) (layer "F.Cu") (net 3))
 (gr_line (start 110 62) (end 108.5 62) (stroke (width 0.2) (type default)) (layer "F.Cu") (net 2))
 (gr_line (start 122 55.5) (end 120.5 54) (stroke (width 0.2) (type default)) (layer "F.Cu") (net 1))
 (gr_line (start 120.5 60) (end 121.5 59) (stroke (width 0.2) (type default)) (layer "F.Cu") (net 1))
 (gr_line (start 124 61) (end 125.5 61) (stroke (width 0.2) (type default)) (layer "B.Cu") (net 4))
 (gr_line (start 120.5 57.5) (end 124 61) (stroke (width 0.2) (type default)) (layer "B.Cu") (net 4))
 (gr_line (start 127 65.5) (end 100 65.5) (stroke (width 0.05) (type default)) (layer "Edge.Cuts"))
 (gr_line (start 127 50) (end 127 65.5) (stroke (width 0.05) (type default)) (layer "Edge.Cuts"))
 (gr_line (start 100 50) (end 100 65.5) (stroke (width 0.05) (type default)) (layer "Edge.Cuts"))
 (gr_line (start 100 50) (end 127 50) (stroke (width 0.05) (type default)) (layer "Edge.Cuts"))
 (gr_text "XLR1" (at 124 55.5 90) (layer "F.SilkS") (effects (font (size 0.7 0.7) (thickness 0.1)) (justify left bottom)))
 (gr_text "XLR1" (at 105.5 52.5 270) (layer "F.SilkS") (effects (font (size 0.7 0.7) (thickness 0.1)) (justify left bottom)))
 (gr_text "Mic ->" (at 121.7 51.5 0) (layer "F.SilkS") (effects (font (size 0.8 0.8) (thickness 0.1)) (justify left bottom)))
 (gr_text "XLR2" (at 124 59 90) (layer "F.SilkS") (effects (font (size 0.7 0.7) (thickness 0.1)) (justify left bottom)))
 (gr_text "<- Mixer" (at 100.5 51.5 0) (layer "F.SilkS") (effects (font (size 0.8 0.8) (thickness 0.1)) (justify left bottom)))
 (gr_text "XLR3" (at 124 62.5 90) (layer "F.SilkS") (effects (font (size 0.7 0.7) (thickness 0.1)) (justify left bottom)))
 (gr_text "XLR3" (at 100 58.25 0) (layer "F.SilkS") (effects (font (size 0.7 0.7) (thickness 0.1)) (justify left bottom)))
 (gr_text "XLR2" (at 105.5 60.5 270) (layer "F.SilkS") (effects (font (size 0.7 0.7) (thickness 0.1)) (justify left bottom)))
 (segment (start 102.6 61.5) (end 102.5 61.6) (width 0.2) (layer "F.Cu") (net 2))
 (segment (start 102.6 62) (end 109 62) (width 0.2) (layer "F.Cu") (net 2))
 (segment (start 117.5 60.5) (end 119 62) (width 0.2) (layer "F.Cu") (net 5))
 (segment (start 121.5 62) (end 120.5 62) (width 0.2) (layer "F.Cu") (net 5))
 (segment (start 116.5625 60.5) (end 117.5 60.5) (width 0.2) (layer "F.Cu") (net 5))
 (segment (start 119 62) (end 120.5 62) (width 0.2) (layer "F.Cu") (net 5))
 (segment (start 125.5 58) (end 121.5 62) (width 0.2) (layer "F.Cu") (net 5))
 (segment (start 119 55) (end 116.0625 55) (width 0.2) (layer "F.Cu") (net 4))
 (segment (start 120.5 57.5) (end 120.5 56) (width 0.2) (layer "F.Cu") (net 4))
 (via (at 120.5 57.5) (size 0.6) (drill 0.3) (layers "F.Cu" "B.Cu") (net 4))
 (segment (start 112.9375 55) (end 110 55) (width 0.2) (layer "F.Cu") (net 3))
 (via (at 108.5 57.5) (size 0.6) (drill 0.3) (layers "F.Cu" "B.Cu") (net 3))
 (segment (start 108 58) (end 102.5 58) (width 0.2) (layer "B.Cu") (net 3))
 (segment (start 108.5 57.5) (end 108 58) (width 0.2) (layer "B.Cu") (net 3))
 (segment (start 110 53) (end 109 54) (width 0.2) (layer "F.Cu") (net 1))
 (segment (start 109 60) (end 108.5 60) (width 0.2) (layer "F.Cu") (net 1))
 (segment (start 109 54) (end 103.4 54) (width 0.2) (layer "F.Cu") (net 1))
 (segment (start 108.5 60) (end 107 58.5) (width 0.2) (layer "F.Cu") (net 1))
 (segment (start 103.4 54) (end 102.9 53.5) (width 0.2) (layer "F.Cu") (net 1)))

